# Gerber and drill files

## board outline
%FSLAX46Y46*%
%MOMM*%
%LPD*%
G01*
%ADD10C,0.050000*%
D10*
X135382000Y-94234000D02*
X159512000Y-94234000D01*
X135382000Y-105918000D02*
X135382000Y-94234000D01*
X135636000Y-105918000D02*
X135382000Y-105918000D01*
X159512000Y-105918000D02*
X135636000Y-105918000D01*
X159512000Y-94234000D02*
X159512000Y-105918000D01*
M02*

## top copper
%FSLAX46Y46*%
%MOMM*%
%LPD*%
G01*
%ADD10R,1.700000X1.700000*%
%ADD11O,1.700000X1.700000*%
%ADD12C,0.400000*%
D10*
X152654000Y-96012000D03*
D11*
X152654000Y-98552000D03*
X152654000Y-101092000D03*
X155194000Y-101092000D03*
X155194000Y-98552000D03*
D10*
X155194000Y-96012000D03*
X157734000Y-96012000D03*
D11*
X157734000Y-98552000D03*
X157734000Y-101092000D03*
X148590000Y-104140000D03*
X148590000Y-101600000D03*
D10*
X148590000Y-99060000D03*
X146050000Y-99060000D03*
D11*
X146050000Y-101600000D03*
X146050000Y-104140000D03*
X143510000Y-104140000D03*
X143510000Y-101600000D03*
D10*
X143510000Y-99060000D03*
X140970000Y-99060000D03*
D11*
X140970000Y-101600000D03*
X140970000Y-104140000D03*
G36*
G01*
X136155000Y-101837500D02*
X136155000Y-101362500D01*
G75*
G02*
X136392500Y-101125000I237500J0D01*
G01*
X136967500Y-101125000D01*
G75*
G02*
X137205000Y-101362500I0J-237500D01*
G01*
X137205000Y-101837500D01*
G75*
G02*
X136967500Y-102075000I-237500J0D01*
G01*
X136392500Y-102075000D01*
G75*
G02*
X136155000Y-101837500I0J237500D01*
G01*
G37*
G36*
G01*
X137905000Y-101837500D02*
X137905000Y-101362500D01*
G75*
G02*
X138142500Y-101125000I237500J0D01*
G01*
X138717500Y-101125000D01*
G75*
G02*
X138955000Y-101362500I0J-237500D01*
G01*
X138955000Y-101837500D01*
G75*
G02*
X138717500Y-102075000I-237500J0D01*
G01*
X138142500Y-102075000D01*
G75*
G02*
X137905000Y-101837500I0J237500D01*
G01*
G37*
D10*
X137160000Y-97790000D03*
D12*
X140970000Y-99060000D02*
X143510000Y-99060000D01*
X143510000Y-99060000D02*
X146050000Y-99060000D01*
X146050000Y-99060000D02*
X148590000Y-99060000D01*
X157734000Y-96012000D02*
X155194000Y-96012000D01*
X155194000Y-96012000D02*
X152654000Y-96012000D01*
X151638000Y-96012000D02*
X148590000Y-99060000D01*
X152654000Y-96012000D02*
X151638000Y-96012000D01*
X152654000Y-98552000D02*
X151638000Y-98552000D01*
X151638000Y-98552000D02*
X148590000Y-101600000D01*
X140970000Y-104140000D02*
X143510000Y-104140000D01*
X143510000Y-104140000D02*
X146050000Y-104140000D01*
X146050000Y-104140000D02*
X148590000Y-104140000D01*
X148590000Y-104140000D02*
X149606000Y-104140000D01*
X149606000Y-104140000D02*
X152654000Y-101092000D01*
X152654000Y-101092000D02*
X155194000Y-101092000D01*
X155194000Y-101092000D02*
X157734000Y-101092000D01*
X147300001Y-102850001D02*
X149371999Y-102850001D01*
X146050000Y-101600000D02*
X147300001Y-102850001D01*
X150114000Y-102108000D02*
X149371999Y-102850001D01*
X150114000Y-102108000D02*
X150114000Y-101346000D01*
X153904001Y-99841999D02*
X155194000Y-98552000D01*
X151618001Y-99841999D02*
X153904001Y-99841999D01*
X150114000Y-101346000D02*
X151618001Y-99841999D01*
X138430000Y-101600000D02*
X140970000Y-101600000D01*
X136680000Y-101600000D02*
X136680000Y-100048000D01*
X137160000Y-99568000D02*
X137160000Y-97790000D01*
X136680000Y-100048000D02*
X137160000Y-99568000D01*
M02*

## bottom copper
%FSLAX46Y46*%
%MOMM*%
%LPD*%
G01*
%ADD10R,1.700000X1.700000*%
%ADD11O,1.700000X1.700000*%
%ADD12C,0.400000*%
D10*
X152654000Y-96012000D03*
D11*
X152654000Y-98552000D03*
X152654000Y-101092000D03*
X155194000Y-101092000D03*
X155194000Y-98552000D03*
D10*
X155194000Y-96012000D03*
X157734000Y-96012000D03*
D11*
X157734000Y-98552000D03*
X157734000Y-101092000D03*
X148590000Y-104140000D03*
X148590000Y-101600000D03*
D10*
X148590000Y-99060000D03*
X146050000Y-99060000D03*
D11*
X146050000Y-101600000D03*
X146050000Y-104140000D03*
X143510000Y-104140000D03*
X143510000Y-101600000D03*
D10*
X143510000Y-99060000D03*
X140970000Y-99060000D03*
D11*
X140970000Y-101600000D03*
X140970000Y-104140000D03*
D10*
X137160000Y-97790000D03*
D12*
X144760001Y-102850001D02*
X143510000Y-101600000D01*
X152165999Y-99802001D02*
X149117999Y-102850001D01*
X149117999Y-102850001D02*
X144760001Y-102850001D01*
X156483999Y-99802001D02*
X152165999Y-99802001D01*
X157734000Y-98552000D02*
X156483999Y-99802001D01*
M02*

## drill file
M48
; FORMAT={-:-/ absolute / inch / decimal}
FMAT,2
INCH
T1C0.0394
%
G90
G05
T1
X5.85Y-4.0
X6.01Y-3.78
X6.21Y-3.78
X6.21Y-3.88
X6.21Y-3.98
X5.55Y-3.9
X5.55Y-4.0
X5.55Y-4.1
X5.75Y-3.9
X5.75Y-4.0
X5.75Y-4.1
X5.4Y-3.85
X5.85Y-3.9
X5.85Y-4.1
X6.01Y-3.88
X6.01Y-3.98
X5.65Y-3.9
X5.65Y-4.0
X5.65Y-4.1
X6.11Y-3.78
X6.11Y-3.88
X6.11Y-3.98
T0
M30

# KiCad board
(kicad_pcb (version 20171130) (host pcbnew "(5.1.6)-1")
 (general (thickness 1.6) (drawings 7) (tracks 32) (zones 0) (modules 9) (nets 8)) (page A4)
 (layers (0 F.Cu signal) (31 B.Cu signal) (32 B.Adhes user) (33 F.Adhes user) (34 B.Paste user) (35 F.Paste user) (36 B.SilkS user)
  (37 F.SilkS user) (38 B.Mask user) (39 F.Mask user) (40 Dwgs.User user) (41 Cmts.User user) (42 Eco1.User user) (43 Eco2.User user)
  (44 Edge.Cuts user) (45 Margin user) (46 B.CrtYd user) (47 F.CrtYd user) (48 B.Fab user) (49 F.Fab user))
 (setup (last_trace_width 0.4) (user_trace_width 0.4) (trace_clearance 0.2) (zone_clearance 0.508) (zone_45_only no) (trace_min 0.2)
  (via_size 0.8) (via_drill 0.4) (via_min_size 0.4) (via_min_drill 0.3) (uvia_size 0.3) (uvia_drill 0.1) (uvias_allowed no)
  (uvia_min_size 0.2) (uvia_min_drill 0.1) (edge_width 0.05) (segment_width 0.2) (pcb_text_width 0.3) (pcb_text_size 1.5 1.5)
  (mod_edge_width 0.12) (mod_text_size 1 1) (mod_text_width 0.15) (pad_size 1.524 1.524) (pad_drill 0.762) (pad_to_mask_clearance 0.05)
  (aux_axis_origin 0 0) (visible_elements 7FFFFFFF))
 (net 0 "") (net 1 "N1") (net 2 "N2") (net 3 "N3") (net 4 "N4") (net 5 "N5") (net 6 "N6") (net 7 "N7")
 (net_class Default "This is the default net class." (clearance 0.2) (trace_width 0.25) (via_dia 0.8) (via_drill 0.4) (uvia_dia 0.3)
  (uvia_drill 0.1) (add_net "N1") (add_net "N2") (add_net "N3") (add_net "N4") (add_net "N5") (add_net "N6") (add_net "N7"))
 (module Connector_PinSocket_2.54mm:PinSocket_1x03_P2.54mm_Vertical (layer B.Cu) (at 152.654 96.012 180)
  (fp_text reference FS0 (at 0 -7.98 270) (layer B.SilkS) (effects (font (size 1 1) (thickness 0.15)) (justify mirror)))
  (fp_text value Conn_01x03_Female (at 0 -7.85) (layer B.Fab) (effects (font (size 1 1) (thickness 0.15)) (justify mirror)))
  (pad 1 thru_hole rect (at 0 0 180) (size 1.7 1.7) (drill 1) (layers *.Cu *.Mask) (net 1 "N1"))
  (pad 2 thru_hole oval (at 0 -2.54 180) (size 1.7 1.7) (drill 1) (layers *.Cu *.Mask) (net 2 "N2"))
  (pad 3 thru_hole oval (at 0 -5.08 180) (size 1.7 1.7) (drill 1) (layers *.Cu *.Mask) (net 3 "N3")))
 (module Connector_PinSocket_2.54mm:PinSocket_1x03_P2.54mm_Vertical (layer B.Cu) (at 155.194 96.012 180)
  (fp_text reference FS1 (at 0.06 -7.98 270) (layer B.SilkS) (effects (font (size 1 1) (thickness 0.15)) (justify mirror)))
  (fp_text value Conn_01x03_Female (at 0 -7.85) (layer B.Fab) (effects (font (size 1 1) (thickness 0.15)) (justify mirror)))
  (pad 3 thru_hole oval (at 0 -5.08 180) (size 1.7 1.7) (drill 1) (layers *.Cu *.Mask) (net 3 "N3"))
  (pad 2 thru_hole oval (at 0 -2.54 180) (size 1.7 1.7) (drill 1) (layers *.Cu *.Mask) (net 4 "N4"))
  (pad 1 thru_hole rect (at 0 0 180) (size 1.7 1.7) (drill 1) (layers *.Cu *.Mask) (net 1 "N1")))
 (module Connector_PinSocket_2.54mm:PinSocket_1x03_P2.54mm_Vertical (layer B.Cu) (at 157.734 96.012 180)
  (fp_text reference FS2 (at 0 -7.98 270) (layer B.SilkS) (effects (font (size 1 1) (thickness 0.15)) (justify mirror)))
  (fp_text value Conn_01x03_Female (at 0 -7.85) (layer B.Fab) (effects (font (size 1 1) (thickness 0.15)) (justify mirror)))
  (pad 1 thru_hole rect (at 0 0 180) (size 1.7 1.7) (drill 1) (layers *.Cu *.Mask) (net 1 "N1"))
  (pad 2 thru_hole oval (at 0 -2.54 180) (size 1.7 1.7) (drill 1) (layers *.Cu *.Mask) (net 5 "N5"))
  (pad 3 thru_hole oval (at 0 -5.08 180) (size 1.7 1.7) (drill 1) (layers *.Cu *.Mask) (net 3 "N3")))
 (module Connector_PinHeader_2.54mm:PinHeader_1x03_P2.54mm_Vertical (layer F.Cu) (at 148.59 99.06)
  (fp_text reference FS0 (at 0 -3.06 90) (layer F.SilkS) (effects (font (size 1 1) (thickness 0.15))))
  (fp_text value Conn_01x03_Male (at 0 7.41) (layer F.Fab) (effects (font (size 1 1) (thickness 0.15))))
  (pad 3 thru_hole oval (at 0 5.08) (size 1.7 1.7) (drill 1) (layers *.Cu *.Mask) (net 3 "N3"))
  (pad 2 thru_hole oval (at 0 2.54) (size 1.7 1.7) (drill 1) (layers *.Cu *.Mask) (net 2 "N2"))
  (pad 1 thru_hole rect (at 0 0) (size 1.7 1.7) (drill 1) (layers *.Cu *.Mask) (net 1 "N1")))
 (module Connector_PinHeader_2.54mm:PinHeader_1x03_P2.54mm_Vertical (layer F.Cu) (at 146.05 99.06)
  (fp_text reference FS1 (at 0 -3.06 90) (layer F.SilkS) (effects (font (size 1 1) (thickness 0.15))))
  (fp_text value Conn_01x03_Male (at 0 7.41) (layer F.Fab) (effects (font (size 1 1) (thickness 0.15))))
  (pad 1 thru_hole rect (at 0 0) (size 1.7 1.7) (drill 1) (layers *.Cu *.Mask) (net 1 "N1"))
  (pad 2 thru_hole oval (at 0 2.54) (size 1.7 1.7) (drill 1) (layers *.Cu *.Mask) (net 4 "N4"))
  (pad 3 thru_hole oval (at 0 5.08) (size 1.7 1.7) (drill 1) (layers *.Cu *.Mask) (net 3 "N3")))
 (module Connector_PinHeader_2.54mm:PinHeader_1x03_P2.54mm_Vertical (layer F.Cu) (at 143.51 99.06)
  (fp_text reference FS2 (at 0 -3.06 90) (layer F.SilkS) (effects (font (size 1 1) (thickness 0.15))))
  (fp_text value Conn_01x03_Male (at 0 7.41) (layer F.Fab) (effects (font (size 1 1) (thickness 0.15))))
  (pad 3 thru_hole oval (at 0 5.08) (size 1.7 1.7) (drill 1) (layers *.Cu *.Mask) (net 3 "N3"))
  (pad 2 thru_hole oval (at 0 2.54) (size 1.7 1.7) (drill 1) (layers *.Cu *.Mask) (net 5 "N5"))
  (pad 1 thru_hole rect (at 0 0) (size 1.7 1.7) (drill 1) (layers *.Cu *.Mask) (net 1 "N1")))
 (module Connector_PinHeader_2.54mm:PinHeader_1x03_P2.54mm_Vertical (layer F.Cu) (at 140.97 99.06)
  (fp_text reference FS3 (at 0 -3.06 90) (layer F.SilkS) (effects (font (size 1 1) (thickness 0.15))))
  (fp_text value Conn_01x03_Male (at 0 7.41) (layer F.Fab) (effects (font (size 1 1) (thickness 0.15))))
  (pad 1 thru_hole rect (at 0 0) (size 1.7 1.7) (drill 1) (layers *.Cu *.Mask) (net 1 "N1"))
  (pad 2 thru_hole oval (at 0 2.54) (size 1.7 1.7) (drill 1) (layers *.Cu *.Mask) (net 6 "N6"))
  (pad 3 thru_hole oval (at 0 5.08) (size 1.7 1.7) (drill 1) (layers *.Cu *.Mask) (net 3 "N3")))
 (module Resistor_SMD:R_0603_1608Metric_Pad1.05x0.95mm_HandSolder (layer F.Cu) (at 137.555 101.6)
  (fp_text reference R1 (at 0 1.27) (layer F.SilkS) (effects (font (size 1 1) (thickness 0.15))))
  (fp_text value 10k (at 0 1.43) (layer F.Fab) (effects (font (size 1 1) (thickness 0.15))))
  (pad 1 smd roundrect (at -0.875 0) (size 1.05 0.95) (layers F.Cu F.Paste F.Mask) (roundrect_rratio 0.25) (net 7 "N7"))
  (pad 2 smd roundrect (at 0.875 0) (size 1.05 0.95) (layers F.Cu F.Paste F.Mask) (roundrect_rratio 0.25) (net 6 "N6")))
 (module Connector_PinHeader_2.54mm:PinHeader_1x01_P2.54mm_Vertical (layer F.Cu) (at 137.16 97.79)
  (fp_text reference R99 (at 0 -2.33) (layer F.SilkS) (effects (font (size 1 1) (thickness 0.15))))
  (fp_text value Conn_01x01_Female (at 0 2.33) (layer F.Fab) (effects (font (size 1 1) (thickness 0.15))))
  (pad 1 thru_hole rect (at 0 0) (size 1.7 1.7) (drill 1) (layers *.Cu *.Mask) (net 7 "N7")))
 (gr_line (start 135.382 94.234) (end 159.512 94.234) (layer Edge.Cuts) (width 0.05))
 (gr_line (start 135.382 105.918) (end 135.382 94.234) (layer Edge.Cuts) (width 0.05))
 (gr_line (start 135.636 105.918) (end 135.382 105.918) (layer Edge.Cuts) (width 0.05))
 (gr_line (start 159.512 105.918) (end 135.636 105.918) (layer Edge.Cuts) (width 0.05))
 (gr_line (start 159.512 94.234) (end 159.512 105.918) (layer Edge.Cuts) (width 0.05))
 (segment (start 140.97 99.06) (end 143.51 99.06) (width 0.4) (layer F.Cu) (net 1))
 (segment (start 143.51 99.06) (end 146.05 99.06) (width 0.4) (layer F.Cu) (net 1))
 (segment (start 146.05 99.06) (end 148.59 99.06) (width 0.4) (layer F.Cu) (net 1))
 (segment (start 157.734 96.012) (end 155.194 96.012) (width 0.4) (layer F.Cu) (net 1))
 (segment (start 155.194 96.012) (end 152.654 96.012) (width 0.4) (layer F.Cu) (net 1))
 (segment (start 151.638 96.012) (end 148.59 99.06) (width 0.4) (layer F.Cu) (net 1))
 (segment (start 152.654 96.012) (end 151.638 96.012) (width 0.4) (layer F.Cu) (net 1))
 (segment (start 152.654 98.552) (end 151.638 98.552) (width 0.4) (layer F.Cu) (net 2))
 (segment (start 151.638 98.552) (end 148.59 101.6) (width 0.4) (layer F.Cu) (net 2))
 (segment (start 140.97 104.14) (end 143.51 104.14) (width 0.4) (layer F.Cu) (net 3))
 (segment (start 143.51 104.14) (end 146.05 104.14) (width 0.4) (layer F.Cu) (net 3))
 (segment (start 146.05 104.14) (end 148.59 104.14) (width 0.4) (layer F.Cu) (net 3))
 (segment (start 148.59 104.14) (end 149.606 104.14) (width 0.4) (layer F.Cu) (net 3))
 (segment (start 149.606 104.14) (end 152.654 101.092) (width 0.4) (layer F.Cu) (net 3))
 (segment (start 152.654 101.092) (end 155.194 101.092) (width 0.4) (layer F.Cu) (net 3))
 (segment (start 155.194 101.092) (end 157.734 101.092) (width 0.4) (layer F.Cu) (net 3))
 (segment (start 147.300001 102.850001) (end 149.371999 102.850001) (width 0.4) (layer F.Cu) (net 4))
 (segment (start 146.05 101.6) (end 147.300001 102.850001) (width 0.4) (layer F.Cu) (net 4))
 (segment (start 150.114 102.108) (end 149.371999 102.850001) (width 0.4) (layer F.Cu) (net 4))
 (segment (start 150.114 102.108) (end 150.114 101.346) (width 0.4) (layer F.Cu) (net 4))
 (segment (start 153.904001 99.841999) (end 155.194 98.552) (width 0.4) (layer F.Cu) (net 4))
 (segment (start 151.618001 99.841999) (end 153.904001 99.841999) (width 0.4) (layer F.Cu) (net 4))
 (segment (start 150.114 101.346) (end 151.618001 99.841999) (width 0.4) (layer F.Cu) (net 4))
 (segment (start 144.760001 102.850001) (end 143.51 101.6) (width 0.4) (layer B.Cu) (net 5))
 (segment (start 152.165999 99.802001) (end 149.117999 102.850001) (width 0.4) (layer B.Cu) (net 5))
 (segment (start 149.117999 102.850001) (end 144.760001 102.850001) (width 0.4) (layer B.Cu) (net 5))
 (segment (start 156.483999 99.802001) (end 152.165999 99.802001) (width 0.4) (layer B.Cu) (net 5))
 (segment (start 157.734 98.552) (end 156.483999 99.802001) (width 0.4) (layer B.Cu) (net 5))
 (segment (start 138.43 101.6) (end 140.97 101.6) (width 0.4) (layer F.Cu) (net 6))
 (segment (start 136.68 101.6) (end 136.68 100.048) (width 0.4) (layer F.Cu) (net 7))
 (segment (start 137.16 99.568) (end 137.16 97.79) (width 0.4) (layer F.Cu) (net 7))
 (segment (start 136.68 100.048) (end 137.16 99.568) (width 0.4) (layer F.Cu) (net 7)))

